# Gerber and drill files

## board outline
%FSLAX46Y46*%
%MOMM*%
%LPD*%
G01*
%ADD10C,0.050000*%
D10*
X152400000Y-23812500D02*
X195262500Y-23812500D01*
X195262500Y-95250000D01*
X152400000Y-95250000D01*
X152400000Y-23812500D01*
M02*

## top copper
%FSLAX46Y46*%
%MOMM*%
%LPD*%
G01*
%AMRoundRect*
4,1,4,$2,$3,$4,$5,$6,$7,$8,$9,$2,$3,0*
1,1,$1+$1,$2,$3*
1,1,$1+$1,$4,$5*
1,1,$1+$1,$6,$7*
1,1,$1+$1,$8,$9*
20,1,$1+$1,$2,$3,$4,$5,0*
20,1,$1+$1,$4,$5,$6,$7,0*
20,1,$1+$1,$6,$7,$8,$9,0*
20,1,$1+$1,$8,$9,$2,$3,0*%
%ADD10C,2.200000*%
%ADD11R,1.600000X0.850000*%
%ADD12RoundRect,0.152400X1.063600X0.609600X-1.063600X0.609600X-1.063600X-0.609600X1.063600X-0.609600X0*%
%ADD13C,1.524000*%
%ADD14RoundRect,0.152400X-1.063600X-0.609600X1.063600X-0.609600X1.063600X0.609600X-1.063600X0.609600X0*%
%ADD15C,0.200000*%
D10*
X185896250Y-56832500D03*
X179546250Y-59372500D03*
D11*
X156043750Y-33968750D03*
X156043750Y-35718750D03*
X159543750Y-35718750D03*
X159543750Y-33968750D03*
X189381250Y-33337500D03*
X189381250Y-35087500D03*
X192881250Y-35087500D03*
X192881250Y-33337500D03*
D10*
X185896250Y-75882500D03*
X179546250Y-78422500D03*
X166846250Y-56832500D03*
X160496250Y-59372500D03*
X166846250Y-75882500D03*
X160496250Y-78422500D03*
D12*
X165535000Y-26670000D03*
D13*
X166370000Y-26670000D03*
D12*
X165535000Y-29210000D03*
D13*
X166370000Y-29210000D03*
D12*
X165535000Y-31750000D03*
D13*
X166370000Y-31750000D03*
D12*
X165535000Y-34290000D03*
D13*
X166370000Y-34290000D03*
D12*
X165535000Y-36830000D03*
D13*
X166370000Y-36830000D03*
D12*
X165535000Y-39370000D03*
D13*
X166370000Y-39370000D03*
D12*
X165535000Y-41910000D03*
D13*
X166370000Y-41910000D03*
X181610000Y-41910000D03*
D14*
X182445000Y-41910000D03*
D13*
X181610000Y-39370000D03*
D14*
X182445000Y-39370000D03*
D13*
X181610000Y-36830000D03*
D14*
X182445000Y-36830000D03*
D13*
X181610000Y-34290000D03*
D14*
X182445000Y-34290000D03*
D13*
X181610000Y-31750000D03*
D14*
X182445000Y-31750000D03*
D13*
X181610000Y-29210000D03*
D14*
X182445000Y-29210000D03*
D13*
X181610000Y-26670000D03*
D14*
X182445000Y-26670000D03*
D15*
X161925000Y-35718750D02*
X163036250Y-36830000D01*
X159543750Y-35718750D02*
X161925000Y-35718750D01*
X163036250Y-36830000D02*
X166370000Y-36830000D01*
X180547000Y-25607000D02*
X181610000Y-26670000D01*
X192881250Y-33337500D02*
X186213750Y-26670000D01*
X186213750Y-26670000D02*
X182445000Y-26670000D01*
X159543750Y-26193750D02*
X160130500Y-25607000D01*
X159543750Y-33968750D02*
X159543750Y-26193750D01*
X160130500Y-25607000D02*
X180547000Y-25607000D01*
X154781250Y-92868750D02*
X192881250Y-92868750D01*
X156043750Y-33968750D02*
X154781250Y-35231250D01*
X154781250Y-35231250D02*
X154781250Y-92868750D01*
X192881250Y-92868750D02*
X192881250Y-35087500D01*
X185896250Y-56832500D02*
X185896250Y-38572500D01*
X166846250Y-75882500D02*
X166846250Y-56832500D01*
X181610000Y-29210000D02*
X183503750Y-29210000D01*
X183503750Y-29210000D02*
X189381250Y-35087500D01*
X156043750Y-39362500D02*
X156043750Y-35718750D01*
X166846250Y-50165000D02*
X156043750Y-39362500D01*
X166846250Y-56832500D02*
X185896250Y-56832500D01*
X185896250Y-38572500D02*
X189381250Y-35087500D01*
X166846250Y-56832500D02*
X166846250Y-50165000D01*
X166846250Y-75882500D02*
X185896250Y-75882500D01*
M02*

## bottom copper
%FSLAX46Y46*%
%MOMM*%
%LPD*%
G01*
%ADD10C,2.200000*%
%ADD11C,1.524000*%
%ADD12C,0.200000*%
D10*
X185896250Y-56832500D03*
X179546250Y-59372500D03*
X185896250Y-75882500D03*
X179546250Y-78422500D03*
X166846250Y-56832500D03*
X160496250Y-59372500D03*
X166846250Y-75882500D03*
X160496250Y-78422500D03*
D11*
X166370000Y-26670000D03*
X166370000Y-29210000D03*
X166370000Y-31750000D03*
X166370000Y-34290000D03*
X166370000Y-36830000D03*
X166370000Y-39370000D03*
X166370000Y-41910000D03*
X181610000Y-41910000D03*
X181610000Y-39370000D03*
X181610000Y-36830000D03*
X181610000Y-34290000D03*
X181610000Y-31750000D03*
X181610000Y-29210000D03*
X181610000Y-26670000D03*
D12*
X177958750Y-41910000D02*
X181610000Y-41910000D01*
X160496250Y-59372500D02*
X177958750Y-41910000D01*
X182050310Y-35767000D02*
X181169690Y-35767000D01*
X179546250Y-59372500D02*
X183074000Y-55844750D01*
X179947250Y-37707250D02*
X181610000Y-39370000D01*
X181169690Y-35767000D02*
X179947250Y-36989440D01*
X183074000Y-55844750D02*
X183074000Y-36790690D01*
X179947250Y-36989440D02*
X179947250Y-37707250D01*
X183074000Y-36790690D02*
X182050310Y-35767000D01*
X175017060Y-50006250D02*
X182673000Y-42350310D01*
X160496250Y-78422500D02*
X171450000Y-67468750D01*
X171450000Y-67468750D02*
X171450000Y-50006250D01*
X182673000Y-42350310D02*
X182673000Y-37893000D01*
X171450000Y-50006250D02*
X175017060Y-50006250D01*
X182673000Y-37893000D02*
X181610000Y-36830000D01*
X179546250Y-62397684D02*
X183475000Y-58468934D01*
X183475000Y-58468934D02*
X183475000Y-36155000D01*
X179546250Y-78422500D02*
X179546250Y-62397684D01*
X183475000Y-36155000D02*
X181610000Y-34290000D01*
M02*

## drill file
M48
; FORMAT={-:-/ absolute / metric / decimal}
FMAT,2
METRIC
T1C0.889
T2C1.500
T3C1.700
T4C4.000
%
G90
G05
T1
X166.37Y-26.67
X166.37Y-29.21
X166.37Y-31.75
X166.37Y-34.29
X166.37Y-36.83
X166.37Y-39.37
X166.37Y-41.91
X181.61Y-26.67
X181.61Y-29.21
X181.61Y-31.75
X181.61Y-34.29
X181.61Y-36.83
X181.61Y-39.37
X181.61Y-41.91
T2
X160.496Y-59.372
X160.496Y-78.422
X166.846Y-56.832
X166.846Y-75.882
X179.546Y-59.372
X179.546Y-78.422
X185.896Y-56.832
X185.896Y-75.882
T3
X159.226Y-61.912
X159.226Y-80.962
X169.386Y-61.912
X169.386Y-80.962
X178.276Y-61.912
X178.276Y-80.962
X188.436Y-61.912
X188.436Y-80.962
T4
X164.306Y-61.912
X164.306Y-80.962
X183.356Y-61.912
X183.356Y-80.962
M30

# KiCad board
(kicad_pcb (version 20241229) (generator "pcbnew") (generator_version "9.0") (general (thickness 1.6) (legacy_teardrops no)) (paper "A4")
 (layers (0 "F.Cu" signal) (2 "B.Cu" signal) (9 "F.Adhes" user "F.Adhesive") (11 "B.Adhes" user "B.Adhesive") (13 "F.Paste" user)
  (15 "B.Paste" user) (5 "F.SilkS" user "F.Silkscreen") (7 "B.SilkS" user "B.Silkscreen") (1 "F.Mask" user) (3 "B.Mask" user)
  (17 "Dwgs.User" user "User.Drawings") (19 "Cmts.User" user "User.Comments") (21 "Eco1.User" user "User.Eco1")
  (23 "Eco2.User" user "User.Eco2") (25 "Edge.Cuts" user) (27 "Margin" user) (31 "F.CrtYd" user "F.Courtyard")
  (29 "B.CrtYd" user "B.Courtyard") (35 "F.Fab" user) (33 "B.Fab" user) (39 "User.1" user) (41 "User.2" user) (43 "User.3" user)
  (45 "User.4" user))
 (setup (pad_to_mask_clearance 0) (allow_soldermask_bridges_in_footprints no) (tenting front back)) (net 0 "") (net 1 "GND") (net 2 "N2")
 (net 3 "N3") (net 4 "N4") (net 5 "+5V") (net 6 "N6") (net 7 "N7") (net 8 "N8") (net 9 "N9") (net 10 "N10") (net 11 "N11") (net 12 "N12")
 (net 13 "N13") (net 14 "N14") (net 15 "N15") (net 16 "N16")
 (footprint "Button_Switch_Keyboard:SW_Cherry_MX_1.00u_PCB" (layer "F.Cu") (at 185.89625 56.8325)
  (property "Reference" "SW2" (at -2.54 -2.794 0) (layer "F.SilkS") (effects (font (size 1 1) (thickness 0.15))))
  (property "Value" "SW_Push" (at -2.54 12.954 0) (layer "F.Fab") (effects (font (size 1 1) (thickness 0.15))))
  (pad "" np_thru_hole circle (at -7.62 5.08) (size 1.7 1.7) (drill 1.7) (layers "*.Cu" "*.Mask"))
  (pad "" np_thru_hole circle (at -2.54 5.08) (size 4 4) (drill 4) (layers "*.Cu" "*.Mask"))
  (pad "" np_thru_hole circle (at 2.54 5.08) (size 1.7 1.7) (drill 1.7) (layers "*.Cu" "*.Mask"))
  (pad "1" thru_hole circle (at 0 0) (size 2.2 2.2) (drill 1.5) (layers "*.Cu" "*.Mask") (remove_unused_layers no) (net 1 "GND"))
  (pad "2" thru_hole circle (at -6.35 2.54) (size 2.2 2.2) (drill 1.5) (layers "*.Cu" "*.Mask") (remove_unused_layers no) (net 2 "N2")))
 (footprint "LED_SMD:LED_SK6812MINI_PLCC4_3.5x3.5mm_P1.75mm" (layer "F.Cu") (at 157.79375 34.84375)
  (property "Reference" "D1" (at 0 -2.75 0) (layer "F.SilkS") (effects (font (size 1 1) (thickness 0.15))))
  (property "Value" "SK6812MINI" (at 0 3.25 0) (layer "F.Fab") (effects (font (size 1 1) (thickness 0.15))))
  (pad "1" smd rect (at -1.75 -0.875) (size 1.6 0.85) (layers "F.Cu" "F.Mask" "F.Paste") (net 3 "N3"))
  (pad "2" smd rect (at -1.75 0.875) (size 1.6 0.85) (layers "F.Cu" "F.Mask" "F.Paste") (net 1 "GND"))
  (pad "3" smd rect (at 1.75 0.875) (size 1.6 0.85) (layers "F.Cu" "F.Mask" "F.Paste") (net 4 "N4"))
  (pad "4" smd rect (at 1.75 -0.875) (size 1.6 0.85) (layers "F.Cu" "F.Mask" "F.Paste") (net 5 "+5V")))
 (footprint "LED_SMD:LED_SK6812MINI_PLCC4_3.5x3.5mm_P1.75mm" (layer "F.Cu") (at 191.13125 34.2125)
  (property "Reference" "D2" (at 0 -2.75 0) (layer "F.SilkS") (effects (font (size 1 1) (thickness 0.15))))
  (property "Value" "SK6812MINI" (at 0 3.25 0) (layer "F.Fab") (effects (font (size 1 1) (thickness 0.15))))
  (pad "1" smd rect (at -1.75 -0.875) (size 1.6 0.85) (layers "F.Cu" "F.Mask" "F.Paste") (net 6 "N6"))
  (pad "2" smd rect (at -1.75 0.875) (size 1.6 0.85) (layers "F.Cu" "F.Mask" "F.Paste") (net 1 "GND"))
  (pad "3" smd rect (at 1.75 0.875) (size 1.6 0.85) (layers "F.Cu" "F.Mask" "F.Paste") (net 3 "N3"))
  (pad "4" smd rect (at 1.75 -0.875) (size 1.6 0.85) (layers "F.Cu" "F.Mask" "F.Paste") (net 5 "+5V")))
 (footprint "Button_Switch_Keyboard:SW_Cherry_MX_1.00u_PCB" (layer "F.Cu") (at 185.89625 75.8825)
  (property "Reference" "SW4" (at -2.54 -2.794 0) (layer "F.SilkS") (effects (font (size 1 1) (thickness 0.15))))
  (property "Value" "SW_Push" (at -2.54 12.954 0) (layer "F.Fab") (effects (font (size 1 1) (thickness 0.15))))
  (pad "" np_thru_hole circle (at -7.62 5.08) (size 1.7 1.7) (drill 1.7) (layers "*.Cu" "*.Mask"))
  (pad "" np_thru_hole circle (at -2.54 5.08) (size 4 4) (drill 4) (layers "*.Cu" "*.Mask"))
  (pad "" np_thru_hole circle (at 2.54 5.08) (size 1.7 1.7) (drill 1.7) (layers "*.Cu" "*.Mask"))
  (pad "1" thru_hole circle (at 0 0) (size 2.2 2.2) (drill 1.5) (layers "*.Cu" "*.Mask") (remove_unused_layers no) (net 1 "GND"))
  (pad "2" thru_hole circle (at -6.35 2.54) (size 2.2 2.2) (drill 1.5) (layers "*.Cu" "*.Mask") (remove_unused_layers no) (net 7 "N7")))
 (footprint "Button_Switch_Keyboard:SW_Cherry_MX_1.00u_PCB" (layer "F.Cu") (at 166.84625 56.8325)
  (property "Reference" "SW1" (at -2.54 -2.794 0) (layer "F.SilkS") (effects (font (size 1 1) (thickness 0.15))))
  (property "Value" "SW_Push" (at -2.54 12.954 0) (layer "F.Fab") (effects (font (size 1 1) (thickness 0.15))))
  (pad "" np_thru_hole circle (at -7.62 5.08) (size 1.7 1.7) (drill 1.7) (layers "*.Cu" "*.Mask"))
  (pad "" np_thru_hole circle (at -2.54 5.08) (size 4 4) (drill 4) (layers "*.Cu" "*.Mask"))
  (pad "" np_thru_hole circle (at 2.54 5.08) (size 1.7 1.7) (drill 1.7) (layers "*.Cu" "*.Mask"))
  (pad "1" thru_hole circle (at 0 0) (size 2.2 2.2) (drill 1.5) (layers "*.Cu" "*.Mask") (remove_unused_layers no) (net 1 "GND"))
  (pad "2" thru_hole circle (at -6.35 2.54) (size 2.2 2.2) (drill 1.5) (layers "*.Cu" "*.Mask") (remove_unused_layers no) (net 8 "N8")))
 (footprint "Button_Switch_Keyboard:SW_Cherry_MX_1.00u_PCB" (layer "F.Cu") (at 166.84625 75.8825)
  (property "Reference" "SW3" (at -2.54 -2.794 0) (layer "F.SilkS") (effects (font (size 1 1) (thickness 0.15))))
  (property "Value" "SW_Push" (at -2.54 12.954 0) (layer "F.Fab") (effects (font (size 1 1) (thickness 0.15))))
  (pad "" np_thru_hole circle (at -7.62 5.08) (size 1.7 1.7) (drill 1.7) (layers "*.Cu" "*.Mask"))
  (pad "" np_thru_hole circle (at -2.54 5.08) (size 4 4) (drill 4) (layers "*.Cu" "*.Mask"))
  (pad "" np_thru_hole circle (at 2.54 5.08) (size 1.7 1.7) (drill 1.7) (layers "*.Cu" "*.Mask"))
  (pad "1" thru_hole circle (at 0 0) (size 2.2 2.2) (drill 1.5) (layers "*.Cu" "*.Mask") (remove_unused_layers no) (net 1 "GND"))
  (pad "2" thru_hole circle (at -6.35 2.54) (size 2.2 2.2) (drill 1.5) (layers "*.Cu" "*.Mask") (remove_unused_layers no) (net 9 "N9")))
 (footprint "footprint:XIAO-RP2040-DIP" (layer "F.Cu") (at 173.99 34.29)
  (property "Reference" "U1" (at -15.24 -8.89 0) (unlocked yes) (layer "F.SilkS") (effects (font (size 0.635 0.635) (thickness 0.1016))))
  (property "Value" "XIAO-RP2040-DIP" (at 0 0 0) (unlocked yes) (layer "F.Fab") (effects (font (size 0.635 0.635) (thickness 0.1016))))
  (pad "1" smd roundrect (at -8.455 -7.62 180) (size 2.432 1.524) (layers "F.Cu" "F.Mask") (roundrect_rratio 0.1) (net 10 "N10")
   (thermal_bridge_angle 45))
  (pad "1" thru_hole circle (at -7.62 -7.62 180) (size 1.524 1.524) (drill 0.889) (layers "*.Cu" "*.Mask") (remove_unused_layers no)
   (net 10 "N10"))
  (pad "2" smd roundrect (at -8.455 -5.08 180) (size 2.432 1.524) (layers "F.Cu" "F.Mask") (roundrect_rratio 0.1) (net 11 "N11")
   (thermal_bridge_angle 45))
  (pad "2" thru_hole circle (at -7.62 -5.08 180) (size 1.524 1.524) (drill 0.889) (layers "*.Cu" "*.Mask") (remove_unused_layers no)
   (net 11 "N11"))
  (pad "3" smd roundrect (at -8.455 -2.54 180) (size 2.432 1.524) (layers "F.Cu" "F.Mask") (roundrect_rratio 0.1) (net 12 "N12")
   (thermal_bridge_angle 45))
  (pad "3" thru_hole circle (at -7.62 -2.54 180) (size 1.524 1.524) (drill 0.889) (layers "*.Cu" "*.Mask") (remove_unused_layers no)
   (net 12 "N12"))
  (pad "4" smd roundrect (at -8.455 0 180) (size 2.432 1.524) (layers "F.Cu" "F.Mask") (roundrect_rratio 0.1) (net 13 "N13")
   (thermal_bridge_angle 45))
  (pad "4" thru_hole circle (at -7.62 0 180) (size 1.524 1.524) (drill 0.889) (layers "*.Cu" "*.Mask") (remove_unused_layers no)
   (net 13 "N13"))
  (pad "5" smd roundrect (at -8.455 2.54 180) (size 2.432 1.524) (layers "F.Cu" "F.Mask") (roundrect_rratio 0.1) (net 4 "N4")
   (thermal_bridge_angle 45))
  (pad "5" thru_hole circle (at -7.62 2.54 180) (size 1.524 1.524) (drill 0.889) (layers "*.Cu" "*.Mask") (remove_unused_layers no)
   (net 4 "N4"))
  (pad "6" smd roundrect (at -8.455 5.08 180) (size 2.432 1.524) (layers "F.Cu" "F.Mask") (roundrect_rratio 0.1) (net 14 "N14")
   (thermal_bridge_angle 45))
  (pad "6" thru_hole circle (at -7.62 5.08 180) (size 1.524 1.524) (drill 0.889) (layers "*.Cu" "*.Mask") (remove_unused_layers no)
   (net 14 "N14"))
  (pad "7" smd roundrect (at -8.455 7.62 180) (size 2.432 1.524) (layers "F.Cu" "F.Mask") (roundrect_rratio 0.1) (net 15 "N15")
   (thermal_bridge_angle 45))
  (pad "7" thru_hole circle (at -7.62 7.62 180) (size 1.524 1.524) (drill 0.889) (layers "*.Cu" "*.Mask") (remove_unused_layers no)
   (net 15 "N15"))
  (pad "8" thru_hole circle (at 7.62 7.62) (size 1.524 1.524) (drill 0.889) (layers "*.Cu" "*.Mask") (remove_unused_layers no) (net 8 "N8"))
  (pad "8" smd roundrect (at 8.455 7.62) (size 2.432 1.524) (layers "F.Cu" "F.Mask") (roundrect_rratio 0.1) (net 8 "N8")
   (thermal_bridge_angle 45))
  (pad "9" thru_hole circle (at 7.62 5.08) (size 1.524 1.524) (drill 0.889) (layers "*.Cu" "*.Mask") (remove_unused_layers no) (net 2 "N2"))
  (pad "9" smd roundrect (at 8.455 5.08) (size 2.432 1.524) (layers "F.Cu" "F.Mask") (roundrect_rratio 0.1) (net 2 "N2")
   (thermal_bridge_angle 45))
  (pad "10" thru_hole circle (at 7.62 2.54) (size 1.524 1.524) (drill 0.889) (layers "*.Cu" "*.Mask") (remove_unused_layers no) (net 9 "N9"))
  (pad "10" smd roundrect (at 8.455 2.54) (size 2.432 1.524) (layers "F.Cu" "F.Mask") (roundrect_rratio 0.1) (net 9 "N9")
   (thermal_bridge_angle 45))
  (pad "11" thru_hole circle (at 7.62 0) (size 1.524 1.524) (drill 0.889) (layers "*.Cu" "*.Mask") (remove_unused_layers no) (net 7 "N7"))
  (pad "11" smd roundrect (at 8.455 0) (size 2.432 1.524) (layers "F.Cu" "F.Mask") (roundrect_rratio 0.1) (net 7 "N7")
   (thermal_bridge_angle 45))
  (pad "12" thru_hole circle (at 7.62 -2.54) (size 1.524 1.524) (drill 0.889) (layers "*.Cu" "*.Mask") (remove_unused_layers no)
   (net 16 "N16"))
  (pad "12" smd roundrect (at 8.455 -2.54) (size 2.432 1.524) (layers "F.Cu" "F.Mask") (roundrect_rratio 0.1) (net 16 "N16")
   (thermal_bridge_angle 45))
  (pad "13" thru_hole circle (at 7.62 -5.08) (size 1.524 1.524) (drill 0.889) (layers "*.Cu" "*.Mask") (remove_unused_layers no)
   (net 1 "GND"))
  (pad "13" smd roundrect (at 8.455 -5.08) (size 2.432 1.524) (layers "F.Cu" "F.Mask") (roundrect_rratio 0.1) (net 1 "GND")
   (thermal_bridge_angle 45))
  (pad "14" thru_hole circle (at 7.62 -7.62) (size 1.524 1.524) (drill 0.889) (layers "*.Cu" "*.Mask") (remove_unused_layers no)
   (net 5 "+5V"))
  (pad "14" smd roundrect (at 8.455 -7.62) (size 2.432 1.524) (layers "F.Cu" "F.Mask") (roundrect_rratio 0.1) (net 5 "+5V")
   (thermal_bridge_angle 45)))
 (gr_rect (start 152.4 23.8125) (end 195.2625 95.25) (stroke (width 0.05) (type default)) (fill no) (layer "Edge.Cuts"))
 (segment (start 161.925 35.71875) (end 163.03625 36.83) (width 0.2) (layer "F.Cu") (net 4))
 (segment (start 159.54375 35.71875) (end 161.925 35.71875) (width 0.2) (layer "F.Cu") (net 4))
 (segment (start 163.03625 36.83) (end 166.37 36.83) (width 0.2) (layer "F.Cu") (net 4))
 (segment (start 180.547 25.607) (end 181.61 26.67) (width 0.2) (layer "F.Cu") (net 5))
 (segment (start 192.88125 33.3375) (end 186.21375 26.67) (width 0.2) (layer "F.Cu") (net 5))
 (segment (start 186.21375 26.67) (end 182.445 26.67) (width 0.2) (layer "F.Cu") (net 5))
 (segment (start 159.54375 26.19375) (end 160.1305 25.607) (width 0.2) (layer "F.Cu") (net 5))
 (segment (start 159.54375 33.96875) (end 159.54375 26.19375) (width 0.2) (layer "F.Cu") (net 5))
 (segment (start 160.1305 25.607) (end 180.547 25.607) (width 0.2) (layer "F.Cu") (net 5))
 (segment (start 154.78125 92.86875) (end 192.88125 92.86875) (width 0.2) (layer "F.Cu") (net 3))
 (segment (start 156.04375 33.96875) (end 154.78125 35.23125) (width 0.2) (layer "F.Cu") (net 3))
 (segment (start 154.78125 35.23125) (end 154.78125 92.86875) (width 0.2) (layer "F.Cu") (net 3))
 (segment (start 192.88125 92.86875) (end 192.88125 35.0875) (width 0.2) (layer "F.Cu") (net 3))
 (segment (start 185.89625 56.8325) (end 185.89625 38.5725) (width 0.2) (layer "F.Cu") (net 1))
 (segment (start 166.84625 75.8825) (end 166.84625 56.8325) (width 0.2) (layer "F.Cu") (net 1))
 (segment (start 181.61 29.21) (end 183.50375 29.21) (width 0.2) (layer "F.Cu") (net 1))
 (segment (start 183.50375 29.21) (end 189.38125 35.0875) (width 0.2) (layer "F.Cu") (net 1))
 (segment (start 156.04375 39.3625) (end 156.04375 35.71875) (width 0.2) (layer "F.Cu") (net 1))
 (segment (start 166.84625 50.165) (end 156.04375 39.3625) (width 0.2) (layer "F.Cu") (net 1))
 (segment (start 166.84625 56.8325) (end 185.89625 56.8325) (width 0.2) (layer "F.Cu") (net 1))
 (segment (start 185.89625 38.5725) (end 189.38125 35.0875) (width 0.2) (layer "F.Cu") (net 1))
 (segment (start 166.84625 56.8325) (end 166.84625 50.165) (width 0.2) (layer "F.Cu") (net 1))
 (segment (start 166.84625 75.8825) (end 185.89625 75.8825) (width 0.2) (layer "F.Cu") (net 1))
 (segment (start 177.95875 41.91) (end 181.61 41.91) (width 0.2) (layer "B.Cu") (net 8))
 (segment (start 160.49625 59.3725) (end 177.95875 41.91) (width 0.2) (layer "B.Cu") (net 8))
 (segment (start 182.05031 35.767) (end 181.16969 35.767) (width 0.2) (layer "B.Cu") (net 2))
 (segment (start 179.54625 59.3725) (end 183.074 55.84475) (width 0.2) (layer "B.Cu") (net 2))
 (segment (start 179.94725 37.70725) (end 181.61 39.37) (width 0.2) (layer "B.Cu") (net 2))
 (segment (start 181.16969 35.767) (end 179.94725 36.98944) (width 0.2) (layer "B.Cu") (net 2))
 (segment (start 183.074 55.84475) (end 183.074 36.79069) (width 0.2) (layer "B.Cu") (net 2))
 (segment (start 179.94725 36.98944) (end 179.94725 37.70725) (width 0.2) (layer "B.Cu") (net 2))
 (segment (start 183.074 36.79069) (end 182.05031 35.767) (width 0.2) (layer "B.Cu") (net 2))
 (segment (start 175.01706 50.00625) (end 182.673 42.35031) (width 0.2) (layer "B.Cu") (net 9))
 (segment (start 160.49625 78.4225) (end 171.45 67.46875) (width 0.2) (layer "B.Cu") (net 9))
 (segment (start 171.45 67.46875) (end 171.45 50.00625) (width 0.2) (layer "B.Cu") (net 9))
 (segment (start 182.673 42.35031) (end 182.673 37.893) (width 0.2) (layer "B.Cu") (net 9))
 (segment (start 171.45 50.00625) (end 175.01706 50.00625) (width 0.2) (layer "B.Cu") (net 9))
 (segment (start 182.673 37.893) (end 181.61 36.83) (width 0.2) (layer "B.Cu") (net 9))
 (segment (start 179.54625 62.397684) (end 183.475 58.468934) (width 0.2) (layer "B.Cu") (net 7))
 (segment (start 183.475 58.468934) (end 183.475 36.155) (width 0.2) (layer "B.Cu") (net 7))
 (segment (start 179.54625 78.4225) (end 179.54625 62.397684) (width 0.2) (layer "B.Cu") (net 7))
 (segment (start 183.475 36.155) (end 181.61 34.29) (width 0.2) (layer "B.Cu") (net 7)))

